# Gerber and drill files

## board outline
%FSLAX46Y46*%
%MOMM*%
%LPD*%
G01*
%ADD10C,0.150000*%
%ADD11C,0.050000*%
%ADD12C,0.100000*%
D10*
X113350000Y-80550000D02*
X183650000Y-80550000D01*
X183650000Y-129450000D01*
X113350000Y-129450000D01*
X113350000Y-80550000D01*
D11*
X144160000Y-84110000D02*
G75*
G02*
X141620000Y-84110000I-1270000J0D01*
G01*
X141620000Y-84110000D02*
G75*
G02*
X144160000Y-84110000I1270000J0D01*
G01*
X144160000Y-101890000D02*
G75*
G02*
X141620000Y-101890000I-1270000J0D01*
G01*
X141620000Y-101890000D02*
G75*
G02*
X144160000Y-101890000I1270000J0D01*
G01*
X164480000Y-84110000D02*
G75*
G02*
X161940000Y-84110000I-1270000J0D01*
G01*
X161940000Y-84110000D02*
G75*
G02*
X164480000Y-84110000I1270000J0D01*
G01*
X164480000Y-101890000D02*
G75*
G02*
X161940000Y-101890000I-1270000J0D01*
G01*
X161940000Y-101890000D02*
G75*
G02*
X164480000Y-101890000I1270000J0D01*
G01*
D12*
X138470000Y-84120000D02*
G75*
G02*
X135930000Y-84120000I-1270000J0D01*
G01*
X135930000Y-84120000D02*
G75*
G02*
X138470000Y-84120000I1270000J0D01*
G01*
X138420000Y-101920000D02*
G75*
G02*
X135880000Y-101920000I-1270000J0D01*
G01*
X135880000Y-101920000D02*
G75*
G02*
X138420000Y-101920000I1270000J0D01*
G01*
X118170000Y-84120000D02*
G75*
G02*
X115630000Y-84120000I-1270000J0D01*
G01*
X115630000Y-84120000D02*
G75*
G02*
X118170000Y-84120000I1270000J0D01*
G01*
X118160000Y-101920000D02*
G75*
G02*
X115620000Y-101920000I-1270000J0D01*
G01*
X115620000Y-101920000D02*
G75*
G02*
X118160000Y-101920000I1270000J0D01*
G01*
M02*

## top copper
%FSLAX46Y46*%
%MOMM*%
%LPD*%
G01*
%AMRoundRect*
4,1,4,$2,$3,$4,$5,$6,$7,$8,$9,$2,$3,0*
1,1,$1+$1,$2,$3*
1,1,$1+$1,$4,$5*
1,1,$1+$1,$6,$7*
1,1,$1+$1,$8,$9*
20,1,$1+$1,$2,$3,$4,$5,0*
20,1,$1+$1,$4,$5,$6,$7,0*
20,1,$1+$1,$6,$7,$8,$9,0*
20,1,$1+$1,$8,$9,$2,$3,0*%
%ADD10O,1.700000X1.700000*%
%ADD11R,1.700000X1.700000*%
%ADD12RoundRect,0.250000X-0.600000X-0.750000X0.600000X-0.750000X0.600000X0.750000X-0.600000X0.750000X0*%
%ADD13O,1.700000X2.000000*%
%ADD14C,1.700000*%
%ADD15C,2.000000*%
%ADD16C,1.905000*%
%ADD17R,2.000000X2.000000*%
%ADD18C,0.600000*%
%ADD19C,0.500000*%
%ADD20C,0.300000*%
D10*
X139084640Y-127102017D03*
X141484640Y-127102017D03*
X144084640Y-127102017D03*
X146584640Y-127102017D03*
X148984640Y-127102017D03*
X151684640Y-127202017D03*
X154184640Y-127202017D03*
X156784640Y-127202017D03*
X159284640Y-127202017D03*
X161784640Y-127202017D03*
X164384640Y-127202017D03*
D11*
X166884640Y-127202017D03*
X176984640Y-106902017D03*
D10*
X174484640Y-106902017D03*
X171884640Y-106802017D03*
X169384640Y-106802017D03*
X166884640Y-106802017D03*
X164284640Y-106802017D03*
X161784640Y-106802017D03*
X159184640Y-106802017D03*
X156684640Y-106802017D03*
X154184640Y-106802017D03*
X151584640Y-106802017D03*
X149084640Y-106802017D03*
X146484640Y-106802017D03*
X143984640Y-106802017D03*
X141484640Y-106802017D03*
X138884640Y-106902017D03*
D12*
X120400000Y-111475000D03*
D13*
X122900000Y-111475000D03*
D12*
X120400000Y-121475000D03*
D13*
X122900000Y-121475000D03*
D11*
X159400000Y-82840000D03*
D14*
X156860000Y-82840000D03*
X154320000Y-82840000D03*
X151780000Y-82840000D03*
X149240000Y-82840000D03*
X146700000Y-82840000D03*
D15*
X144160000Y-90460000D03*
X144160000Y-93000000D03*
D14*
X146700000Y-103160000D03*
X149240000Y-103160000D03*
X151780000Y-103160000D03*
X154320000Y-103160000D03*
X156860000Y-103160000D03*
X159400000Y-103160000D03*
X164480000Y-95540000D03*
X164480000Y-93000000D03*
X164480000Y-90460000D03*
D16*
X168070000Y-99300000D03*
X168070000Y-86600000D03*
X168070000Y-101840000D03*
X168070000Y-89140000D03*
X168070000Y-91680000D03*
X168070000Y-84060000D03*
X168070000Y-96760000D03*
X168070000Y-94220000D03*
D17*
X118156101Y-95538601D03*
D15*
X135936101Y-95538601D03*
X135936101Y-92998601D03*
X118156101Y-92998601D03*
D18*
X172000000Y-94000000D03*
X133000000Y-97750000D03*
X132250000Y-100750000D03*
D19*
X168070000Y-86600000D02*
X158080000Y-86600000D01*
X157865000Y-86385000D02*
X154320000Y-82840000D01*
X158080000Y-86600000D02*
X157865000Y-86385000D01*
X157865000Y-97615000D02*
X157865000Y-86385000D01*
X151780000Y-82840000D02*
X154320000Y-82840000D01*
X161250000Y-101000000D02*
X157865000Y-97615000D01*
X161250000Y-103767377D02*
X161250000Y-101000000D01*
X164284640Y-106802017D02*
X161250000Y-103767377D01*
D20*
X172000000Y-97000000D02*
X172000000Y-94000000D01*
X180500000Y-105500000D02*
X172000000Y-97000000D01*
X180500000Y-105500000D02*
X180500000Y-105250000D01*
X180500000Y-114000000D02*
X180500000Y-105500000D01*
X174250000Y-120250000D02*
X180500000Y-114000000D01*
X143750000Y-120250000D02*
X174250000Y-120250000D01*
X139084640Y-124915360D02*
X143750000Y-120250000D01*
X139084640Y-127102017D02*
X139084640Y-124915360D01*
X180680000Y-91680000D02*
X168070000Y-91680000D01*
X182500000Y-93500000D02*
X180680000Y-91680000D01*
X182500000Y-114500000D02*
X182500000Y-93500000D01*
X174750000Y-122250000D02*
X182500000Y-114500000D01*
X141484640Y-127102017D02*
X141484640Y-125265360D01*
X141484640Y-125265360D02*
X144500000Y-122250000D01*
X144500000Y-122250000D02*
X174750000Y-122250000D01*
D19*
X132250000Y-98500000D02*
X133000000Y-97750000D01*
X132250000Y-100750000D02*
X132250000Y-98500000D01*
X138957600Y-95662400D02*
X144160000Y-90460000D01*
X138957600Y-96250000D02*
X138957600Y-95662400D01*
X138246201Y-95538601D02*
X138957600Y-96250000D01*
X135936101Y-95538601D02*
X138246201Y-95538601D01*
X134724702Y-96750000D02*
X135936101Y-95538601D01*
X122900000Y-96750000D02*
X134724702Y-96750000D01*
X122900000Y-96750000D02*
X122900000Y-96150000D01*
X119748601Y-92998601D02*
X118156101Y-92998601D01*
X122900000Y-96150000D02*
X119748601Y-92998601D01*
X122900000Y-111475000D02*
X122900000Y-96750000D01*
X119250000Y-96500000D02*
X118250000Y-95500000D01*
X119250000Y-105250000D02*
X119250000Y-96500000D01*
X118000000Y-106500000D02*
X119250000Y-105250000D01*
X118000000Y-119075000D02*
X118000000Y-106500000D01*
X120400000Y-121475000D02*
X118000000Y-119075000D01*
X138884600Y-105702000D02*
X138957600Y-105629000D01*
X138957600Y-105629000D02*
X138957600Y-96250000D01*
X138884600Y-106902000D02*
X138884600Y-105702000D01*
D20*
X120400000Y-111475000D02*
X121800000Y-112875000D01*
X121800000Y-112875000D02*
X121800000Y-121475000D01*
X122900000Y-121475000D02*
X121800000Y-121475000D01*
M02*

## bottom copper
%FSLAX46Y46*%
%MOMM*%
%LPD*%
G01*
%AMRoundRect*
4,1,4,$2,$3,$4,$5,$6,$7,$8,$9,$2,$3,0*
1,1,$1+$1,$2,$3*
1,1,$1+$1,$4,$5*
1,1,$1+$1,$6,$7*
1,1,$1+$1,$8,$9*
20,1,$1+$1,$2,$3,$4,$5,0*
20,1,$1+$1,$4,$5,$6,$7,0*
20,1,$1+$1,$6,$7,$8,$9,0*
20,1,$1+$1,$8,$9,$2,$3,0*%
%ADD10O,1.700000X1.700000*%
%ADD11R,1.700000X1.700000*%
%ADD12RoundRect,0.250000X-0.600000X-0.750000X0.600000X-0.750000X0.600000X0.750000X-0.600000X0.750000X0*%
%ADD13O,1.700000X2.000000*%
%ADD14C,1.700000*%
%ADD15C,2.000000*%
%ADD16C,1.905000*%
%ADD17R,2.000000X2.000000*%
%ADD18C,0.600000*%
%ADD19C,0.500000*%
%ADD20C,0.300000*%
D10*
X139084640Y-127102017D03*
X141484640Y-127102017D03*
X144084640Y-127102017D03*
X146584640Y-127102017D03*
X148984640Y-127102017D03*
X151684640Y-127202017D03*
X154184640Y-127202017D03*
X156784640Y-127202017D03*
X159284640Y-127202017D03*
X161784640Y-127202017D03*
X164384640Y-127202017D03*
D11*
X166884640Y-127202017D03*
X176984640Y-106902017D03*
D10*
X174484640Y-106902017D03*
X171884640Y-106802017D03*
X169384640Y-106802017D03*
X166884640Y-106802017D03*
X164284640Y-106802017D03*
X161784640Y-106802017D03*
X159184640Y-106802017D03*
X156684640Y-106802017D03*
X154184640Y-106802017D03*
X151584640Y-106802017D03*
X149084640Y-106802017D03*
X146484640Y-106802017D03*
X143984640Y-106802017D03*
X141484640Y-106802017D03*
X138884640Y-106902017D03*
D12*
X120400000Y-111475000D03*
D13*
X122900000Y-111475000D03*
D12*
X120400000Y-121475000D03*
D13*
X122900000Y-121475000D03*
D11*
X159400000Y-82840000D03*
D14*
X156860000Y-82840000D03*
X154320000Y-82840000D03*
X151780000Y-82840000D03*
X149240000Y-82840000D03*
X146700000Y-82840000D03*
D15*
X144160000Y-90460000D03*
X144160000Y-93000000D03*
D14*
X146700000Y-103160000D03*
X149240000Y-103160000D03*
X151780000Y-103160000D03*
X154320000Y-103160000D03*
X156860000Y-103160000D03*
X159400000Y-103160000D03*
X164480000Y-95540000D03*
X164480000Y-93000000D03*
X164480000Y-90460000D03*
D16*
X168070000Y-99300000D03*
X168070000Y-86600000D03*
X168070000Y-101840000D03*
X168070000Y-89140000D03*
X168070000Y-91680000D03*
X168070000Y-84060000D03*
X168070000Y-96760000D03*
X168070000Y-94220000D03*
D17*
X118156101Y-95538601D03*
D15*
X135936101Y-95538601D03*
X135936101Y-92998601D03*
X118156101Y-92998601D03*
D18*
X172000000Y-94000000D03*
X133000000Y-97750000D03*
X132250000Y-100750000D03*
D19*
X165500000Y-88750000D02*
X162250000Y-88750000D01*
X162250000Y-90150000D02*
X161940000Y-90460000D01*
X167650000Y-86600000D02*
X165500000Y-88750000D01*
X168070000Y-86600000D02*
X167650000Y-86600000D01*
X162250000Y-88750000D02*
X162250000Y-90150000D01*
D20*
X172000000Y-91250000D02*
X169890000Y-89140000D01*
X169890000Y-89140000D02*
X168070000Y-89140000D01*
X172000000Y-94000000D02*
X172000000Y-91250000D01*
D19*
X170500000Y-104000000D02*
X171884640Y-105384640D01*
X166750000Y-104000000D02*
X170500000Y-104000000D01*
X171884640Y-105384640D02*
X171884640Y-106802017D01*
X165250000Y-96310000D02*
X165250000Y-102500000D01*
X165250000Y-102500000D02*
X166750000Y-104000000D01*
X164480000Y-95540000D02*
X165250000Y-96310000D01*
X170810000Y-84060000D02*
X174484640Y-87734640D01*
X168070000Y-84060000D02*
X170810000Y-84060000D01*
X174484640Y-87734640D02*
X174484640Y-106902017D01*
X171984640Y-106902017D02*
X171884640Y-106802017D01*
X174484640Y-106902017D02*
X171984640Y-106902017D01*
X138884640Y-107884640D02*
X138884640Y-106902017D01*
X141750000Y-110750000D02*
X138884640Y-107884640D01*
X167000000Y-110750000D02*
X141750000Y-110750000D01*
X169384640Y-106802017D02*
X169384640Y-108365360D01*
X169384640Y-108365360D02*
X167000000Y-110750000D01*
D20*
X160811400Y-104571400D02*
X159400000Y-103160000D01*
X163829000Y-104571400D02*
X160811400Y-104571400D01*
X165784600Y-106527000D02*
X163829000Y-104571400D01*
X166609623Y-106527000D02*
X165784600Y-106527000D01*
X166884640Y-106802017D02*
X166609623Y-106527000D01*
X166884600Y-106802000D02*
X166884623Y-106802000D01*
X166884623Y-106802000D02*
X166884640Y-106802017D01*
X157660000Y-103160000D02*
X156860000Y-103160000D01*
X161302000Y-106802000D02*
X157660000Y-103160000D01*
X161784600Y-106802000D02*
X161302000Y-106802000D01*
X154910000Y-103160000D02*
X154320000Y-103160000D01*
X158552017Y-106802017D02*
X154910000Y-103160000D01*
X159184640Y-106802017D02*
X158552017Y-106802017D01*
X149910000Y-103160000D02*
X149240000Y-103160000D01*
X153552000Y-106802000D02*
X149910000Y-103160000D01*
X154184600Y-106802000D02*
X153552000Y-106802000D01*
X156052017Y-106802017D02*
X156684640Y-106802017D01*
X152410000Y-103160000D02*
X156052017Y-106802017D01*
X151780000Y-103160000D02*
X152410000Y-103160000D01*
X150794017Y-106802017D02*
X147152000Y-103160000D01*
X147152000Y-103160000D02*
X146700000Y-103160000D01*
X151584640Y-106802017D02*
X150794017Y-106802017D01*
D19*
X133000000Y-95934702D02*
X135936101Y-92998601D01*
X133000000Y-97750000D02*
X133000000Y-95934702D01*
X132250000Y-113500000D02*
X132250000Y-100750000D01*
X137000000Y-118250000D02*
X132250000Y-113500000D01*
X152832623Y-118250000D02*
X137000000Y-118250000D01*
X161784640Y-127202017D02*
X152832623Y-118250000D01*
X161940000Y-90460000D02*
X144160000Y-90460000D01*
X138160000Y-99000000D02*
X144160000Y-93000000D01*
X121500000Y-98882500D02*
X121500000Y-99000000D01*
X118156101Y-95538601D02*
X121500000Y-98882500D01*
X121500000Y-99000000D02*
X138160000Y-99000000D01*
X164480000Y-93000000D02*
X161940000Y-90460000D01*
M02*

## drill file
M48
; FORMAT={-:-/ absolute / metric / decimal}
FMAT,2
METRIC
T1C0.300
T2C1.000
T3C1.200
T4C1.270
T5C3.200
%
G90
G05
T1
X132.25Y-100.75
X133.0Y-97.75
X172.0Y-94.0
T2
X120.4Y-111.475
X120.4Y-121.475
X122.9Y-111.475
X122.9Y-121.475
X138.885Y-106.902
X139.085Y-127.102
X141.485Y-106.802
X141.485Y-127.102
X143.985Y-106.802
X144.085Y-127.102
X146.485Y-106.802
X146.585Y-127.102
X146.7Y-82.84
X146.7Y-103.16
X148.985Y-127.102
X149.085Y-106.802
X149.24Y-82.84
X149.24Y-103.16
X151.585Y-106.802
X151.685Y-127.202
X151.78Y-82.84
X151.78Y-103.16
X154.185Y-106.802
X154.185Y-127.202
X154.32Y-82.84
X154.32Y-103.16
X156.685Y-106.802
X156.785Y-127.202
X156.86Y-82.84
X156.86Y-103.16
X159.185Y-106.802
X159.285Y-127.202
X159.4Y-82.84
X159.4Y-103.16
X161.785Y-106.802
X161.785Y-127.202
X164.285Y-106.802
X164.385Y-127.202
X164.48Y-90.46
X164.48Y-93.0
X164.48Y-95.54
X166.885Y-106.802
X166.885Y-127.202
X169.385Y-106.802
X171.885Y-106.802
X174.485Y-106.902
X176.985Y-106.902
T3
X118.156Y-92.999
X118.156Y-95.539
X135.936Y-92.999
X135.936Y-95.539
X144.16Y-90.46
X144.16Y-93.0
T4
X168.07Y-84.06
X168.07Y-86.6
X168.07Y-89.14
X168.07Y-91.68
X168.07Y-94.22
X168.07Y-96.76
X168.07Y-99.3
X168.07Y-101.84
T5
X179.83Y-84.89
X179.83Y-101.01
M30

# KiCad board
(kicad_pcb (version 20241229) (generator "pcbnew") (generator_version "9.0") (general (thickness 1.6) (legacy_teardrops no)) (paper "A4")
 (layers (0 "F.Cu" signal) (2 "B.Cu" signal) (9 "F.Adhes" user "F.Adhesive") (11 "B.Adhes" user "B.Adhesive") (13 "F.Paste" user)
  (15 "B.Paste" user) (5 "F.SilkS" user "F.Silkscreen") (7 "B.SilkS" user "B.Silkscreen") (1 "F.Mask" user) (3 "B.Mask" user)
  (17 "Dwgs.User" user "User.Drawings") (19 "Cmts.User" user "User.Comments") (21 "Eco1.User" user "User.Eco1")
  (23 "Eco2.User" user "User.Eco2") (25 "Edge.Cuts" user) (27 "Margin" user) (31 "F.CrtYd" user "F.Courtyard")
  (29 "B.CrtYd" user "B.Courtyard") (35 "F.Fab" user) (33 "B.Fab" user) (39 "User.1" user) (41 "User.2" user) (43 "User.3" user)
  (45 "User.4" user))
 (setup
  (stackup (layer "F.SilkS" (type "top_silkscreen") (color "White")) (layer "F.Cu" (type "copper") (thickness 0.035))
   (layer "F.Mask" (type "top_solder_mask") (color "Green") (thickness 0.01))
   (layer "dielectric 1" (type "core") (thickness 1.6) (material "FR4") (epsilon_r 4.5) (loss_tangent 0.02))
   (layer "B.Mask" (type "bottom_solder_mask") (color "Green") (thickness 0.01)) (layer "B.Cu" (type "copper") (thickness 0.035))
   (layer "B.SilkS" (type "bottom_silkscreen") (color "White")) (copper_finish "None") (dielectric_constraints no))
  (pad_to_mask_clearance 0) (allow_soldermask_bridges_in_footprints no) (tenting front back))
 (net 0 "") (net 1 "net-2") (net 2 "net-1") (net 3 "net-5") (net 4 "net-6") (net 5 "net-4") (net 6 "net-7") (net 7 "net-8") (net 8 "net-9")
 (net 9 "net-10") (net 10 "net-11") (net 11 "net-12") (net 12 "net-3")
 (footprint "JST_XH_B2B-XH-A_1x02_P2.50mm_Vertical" (layer "F.Cu") (at 121.65 112)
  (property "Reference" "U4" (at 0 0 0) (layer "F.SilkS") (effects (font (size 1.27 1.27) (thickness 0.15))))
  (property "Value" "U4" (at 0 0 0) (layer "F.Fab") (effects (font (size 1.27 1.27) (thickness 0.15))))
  (pad "1" thru_hole roundrect (at -1.25 -0.525) (size 1.7 2) (drill 1) (layers "*.Cu" "*.Mask") (remove_unused_layers no)
   (roundrect_rratio 0.147059) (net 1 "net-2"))
  (pad "2" thru_hole oval (at 1.25 -0.525) (size 1.7 2) (drill 1) (layers "*.Cu" "*.Mask") (remove_unused_layers no) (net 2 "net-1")))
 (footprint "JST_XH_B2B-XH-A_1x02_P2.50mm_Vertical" (layer "F.Cu") (at 121.65 122)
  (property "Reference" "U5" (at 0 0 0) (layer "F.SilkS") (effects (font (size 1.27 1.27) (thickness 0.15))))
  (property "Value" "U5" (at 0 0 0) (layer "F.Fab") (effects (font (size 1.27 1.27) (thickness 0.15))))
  (pad "1" thru_hole roundrect (at -1.25 -0.525) (size 1.7 2) (drill 1) (layers "*.Cu" "*.Mask") (remove_unused_layers no)
   (roundrect_rratio 0.147059) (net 2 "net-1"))
  (pad "2" thru_hole oval (at 1.25 -0.525) (size 1.7 2) (drill 1) (layers "*.Cu" "*.Mask") (remove_unused_layers no) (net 1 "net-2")))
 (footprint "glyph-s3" (layer "F.Cu") (at 157.978 117.1 180)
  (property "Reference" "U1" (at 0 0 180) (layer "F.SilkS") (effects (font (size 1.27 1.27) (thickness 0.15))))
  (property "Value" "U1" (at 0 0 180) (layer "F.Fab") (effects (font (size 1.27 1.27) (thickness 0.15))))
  (pad "1" thru_hole oval (at 18.89336 -10.002017 270) (size 1.7 1.7) (drill 1) (layers "*.Cu" "*.Mask") (remove_unused_layers no))
  (pad "2" thru_hole oval (at 16.49336 -10.002017 270) (size 1.7 1.7) (drill 1) (layers "*.Cu" "*.Mask") (remove_unused_layers no))
  (pad "3" thru_hole oval (at 13.89336 -10.002017 270) (size 1.7 1.7) (drill 1) (layers "*.Cu" "*.Mask") (remove_unused_layers no)
   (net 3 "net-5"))
  (pad "4" thru_hole oval (at 11.39336 -10.002017 270) (size 1.7 1.7) (drill 1) (layers "*.Cu" "*.Mask") (remove_unused_layers no)
   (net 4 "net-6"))
  (pad "5" thru_hole oval (at 8.99336 -10.002017 270) (size 1.7 1.7) (drill 1) (layers "*.Cu" "*.Mask") (remove_unused_layers no))
  (pad "6" thru_hole oval (at 6.29336 -10.102017 270) (size 1.7 1.7) (drill 1) (layers "*.Cu" "*.Mask") (remove_unused_layers no))
  (pad "7" thru_hole oval (at 3.79336 -10.102017 270) (size 1.7 1.7) (drill 1) (layers "*.Cu" "*.Mask") (remove_unused_layers no))
  (pad "8" thru_hole oval (at 1.19336 -10.102017 270) (size 1.7 1.7) (drill 1) (layers "*.Cu" "*.Mask") (remove_unused_layers no))
  (pad "9" thru_hole oval (at -1.30664 -10.102017 270) (size 1.7 1.7) (drill 1) (layers "*.Cu" "*.Mask") (remove_unused_layers no))
  (pad "10" thru_hole oval (at -3.80664 -10.102017 270) (size 1.7 1.7) (drill 1) (layers "*.Cu" "*.Mask") (remove_unused_layers no)
   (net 2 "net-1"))
  (pad "11" thru_hole oval (at -6.40664 -10.102017 270) (size 1.7 1.7) (drill 1) (layers "*.Cu" "*.Mask") (remove_unused_layers no))
  (pad "12" thru_hole rect (at -8.90664 -10.102017 270) (size 1.7 1.7) (drill 1) (layers "*.Cu" "*.Mask") (remove_unused_layers no))
  (pad "13" thru_hole rect (at -19.00664 10.197983 270) (size 1.7 1.7) (drill 1) (layers "*.Cu" "*.Mask") (remove_unused_layers no))
  (pad "14" thru_hole oval (at -16.50664 10.197983 270) (size 1.7 1.7) (drill 1) (layers "*.Cu" "*.Mask") (remove_unused_layers no)
   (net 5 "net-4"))
  (pad "15" thru_hole oval (at -13.90664 10.297983 270) (size 1.7 1.7) (drill 1) (layers "*.Cu" "*.Mask") (remove_unused_layers no)
   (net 5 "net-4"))
  (pad "16" thru_hole oval (at -11.40664 10.297983 270) (size 1.7 1.7) (drill 1) (layers "*.Cu" "*.Mask") (remove_unused_layers no)
   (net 2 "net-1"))
  (pad "17" thru_hole oval (at -8.90664 10.297983 270) (size 1.7 1.7) (drill 1) (layers "*.Cu" "*.Mask") (remove_unused_layers no)
   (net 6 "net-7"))
  (pad "18" thru_hole oval (at -6.30664 10.297983 270) (size 1.7 1.7) (drill 1) (layers "*.Cu" "*.Mask") (remove_unused_layers no))
  (pad "19" thru_hole oval (at -3.80664 10.297983 270) (size 1.7 1.7) (drill 1) (layers "*.Cu" "*.Mask") (remove_unused_layers no)
   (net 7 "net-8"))
  (pad "20" thru_hole oval (at -1.20664 10.297983 270) (size 1.7 1.7) (drill 1) (layers "*.Cu" "*.Mask") (remove_unused_layers no)
   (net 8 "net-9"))
  (pad "21" thru_hole oval (at 1.29336 10.297983 270) (size 1.7 1.7) (drill 1) (layers "*.Cu" "*.Mask") (remove_unused_layers no)
   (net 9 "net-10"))
  (pad "22" thru_hole oval (at 3.79336 10.297983 270) (size 1.7 1.7) (drill 1) (layers "*.Cu" "*.Mask") (remove_unused_layers no)
   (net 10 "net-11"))
  (pad "23" thru_hole oval (at 6.39336 10.297983 270) (size 1.7 1.7) (drill 1) (layers "*.Cu" "*.Mask") (remove_unused_layers no)
   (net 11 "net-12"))
  (pad "24" thru_hole oval (at 8.89336 10.297983 270) (size 1.7 1.7) (drill 1) (layers "*.Cu" "*.Mask") (remove_unused_layers no))
  (pad "25" thru_hole oval (at 11.49336 10.297983 270) (size 1.7 1.7) (drill 1) (layers "*.Cu" "*.Mask") (remove_unused_layers no))
  (pad "26" thru_hole oval (at 13.99336 10.297983 270) (size 1.7 1.7) (drill 1) (layers "*.Cu" "*.Mask") (remove_unused_layers no))
  (pad "27" thru_hole oval (at 16.49336 10.297983 270) (size 1.7 1.7) (drill 1) (layers "*.Cu" "*.Mask") (remove_unused_layers no))
  (pad "28" thru_hole oval (at 19.09336 10.197983 270) (size 1.7 1.7) (drill 1) (layers "*.Cu" "*.Mask") (remove_unused_layers no)
   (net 2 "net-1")))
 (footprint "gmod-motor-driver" (layer "F.Cu") (at 153.05 93)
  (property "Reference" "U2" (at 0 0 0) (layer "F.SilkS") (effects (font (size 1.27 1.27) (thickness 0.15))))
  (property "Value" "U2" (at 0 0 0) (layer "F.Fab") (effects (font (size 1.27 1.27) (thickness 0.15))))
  (fp_circle (center -10.16 -8.89) (end -10.16 -10.16) (stroke (width 0.05) (type default)) (fill no) (layer "Edge.Cuts"))
  (fp_circle (center -10.16 8.89) (end -10.16 7.62) (stroke (width 0.05) (type default)) (fill no) (layer "Edge.Cuts"))
  (fp_circle (center 10.16 -8.89) (end 10.16 -10.16) (stroke (width 0.05) (type default)) (fill no) (layer "Edge.Cuts"))
  (fp_circle (center 10.16 8.89) (end 10.16 7.62) (stroke (width 0.05) (type default)) (fill no) (layer "Edge.Cuts"))
  (pad "1" thru_hole rect (at 6.35 -10.16 270) (size 1.7 1.7) (drill 1) (layers "*.Cu" "*.Mask") (remove_unused_layers no))
  (pad "2" thru_hole circle (at 3.81 -10.16 270) (size 1.7 1.7) (drill 1) (layers "*.Cu" "*.Mask") (remove_unused_layers no))
  (pad "3" thru_hole circle (at 1.27 -10.16 270) (size 1.7 1.7) (drill 1) (layers "*.Cu" "*.Mask") (remove_unused_layers no))
  (pad "4" thru_hole circle (at -1.27 -10.16 270) (size 1.7 1.7) (drill 1) (layers "*.Cu" "*.Mask") (remove_unused_layers no))
  (pad "5" thru_hole circle (at -3.81 -10.16 270) (size 1.7 1.7) (drill 1) (layers "*.Cu" "*.Mask") (remove_unused_layers no))
  (pad "6" thru_hole circle (at -6.35 -10.16 270) (size 1.7 1.7) (drill 1) (layers "*.Cu" "*.Mask") (remove_unused_layers no))
  (pad "7" thru_hole circle (at -8.89 -2.54 270) (size 2 2) (drill 1.2) (layers "*.Cu" "*.Mask") (remove_unused_layers no) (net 2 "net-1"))
  (pad "8" thru_hole circle (at -8.89 0 270) (size 2 2) (drill 1.2) (layers "*.Cu" "*.Mask") (remove_unused_layers no) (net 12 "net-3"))
  (pad "9" thru_hole circle (at -6.35 10.16 270) (size 1.7 1.7) (drill 1) (layers "*.Cu" "*.Mask") (remove_unused_layers no)
   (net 11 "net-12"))
  (pad "10" thru_hole circle (at -3.81 10.16 270) (size 1.7 1.7) (drill 1) (layers "*.Cu" "*.Mask") (remove_unused_layers no)
   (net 10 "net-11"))
  (pad "11" thru_hole circle (at -1.27 10.16 270) (size 1.7 1.7) (drill 1) (layers "*.Cu" "*.Mask") (remove_unused_layers no)
   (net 9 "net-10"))
  (pad "12" thru_hole circle (at 1.27 10.16 270) (size 1.7 1.7) (drill 1) (layers "*.Cu" "*.Mask") (remove_unused_layers no) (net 8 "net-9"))
  (pad "13" thru_hole circle (at 3.81 10.16 270) (size 1.7 1.7) (drill 1) (layers "*.Cu" "*.Mask") (remove_unused_layers no) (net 7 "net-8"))
  (pad "14" thru_hole circle (at 6.35 10.16 270) (size 1.7 1.7) (drill 1) (layers "*.Cu" "*.Mask") (remove_unused_layers no) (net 6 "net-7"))
  (pad "15" thru_hole circle (at 11.43 2.54 180) (size 1.7 1.7) (drill 1) (layers "*.Cu" "*.Mask") (remove_unused_layers no) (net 5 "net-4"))
  (pad "16" thru_hole circle (at 11.43 0 180) (size 1.7 1.7) (drill 1) (layers "*.Cu" "*.Mask") (remove_unused_layers no) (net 2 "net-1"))
  (pad "17" thru_hole circle (at 11.43 -2.54 180) (size 1.7 1.7) (drill 1) (layers "*.Cu" "*.Mask") (remove_unused_layers no)))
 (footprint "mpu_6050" (layer "F.Cu") (at 174.4 92.95)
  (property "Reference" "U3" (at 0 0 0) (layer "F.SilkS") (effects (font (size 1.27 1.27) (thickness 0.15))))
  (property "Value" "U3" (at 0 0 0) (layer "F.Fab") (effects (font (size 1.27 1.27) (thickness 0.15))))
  (pad "" np_thru_hole circle (at 5.43 -8.06) (size 3.2 3.2) (drill 3.2) (layers "*.Cu" "*.Mask"))
  (pad "" np_thru_hole circle (at 5.43 8.06) (size 3.2 3.2) (drill 3.2) (layers "*.Cu" "*.Mask"))
  (pad "AD0" thru_hole circle (at -6.33 6.35) (size 1.905 1.905) (drill 1.27) (layers "*.Cu" "*.Mask") (remove_unused_layers no)
   (solder_mask_margin 0.102))
  (pad "GND" thru_hole circle (at -6.33 -6.35) (size 1.905 1.905) (drill 1.27) (layers "*.Cu" "*.Mask") (remove_unused_layers no)
   (solder_mask_margin 0.102))
  (pad "INT" thru_hole circle (at -6.33 8.89) (size 1.905 1.905) (drill 1.27) (layers "*.Cu" "*.Mask") (remove_unused_layers no)
   (solder_mask_margin 0.102))
  (pad "SCL" thru_hole circle (at -6.33 -3.81) (size 1.905 1.905) (drill 1.27) (layers "*.Cu" "*.Mask") (remove_unused_layers no)
   (solder_mask_margin 0.102))
  (pad "SDA" thru_hole circle (at -6.33 -1.27) (size 1.905 1.905) (drill 1.27) (layers "*.Cu" "*.Mask") (remove_unused_layers no)
   (solder_mask_margin 0.102))
  (pad "VCC" thru_hole circle (at -6.33 -8.89) (size 1.905 1.905) (drill 1.27) (layers "*.Cu" "*.Mask") (remove_unused_layers no)
   (solder_mask_margin 0.102))
  (pad "XCL" thru_hole circle (at -6.33 3.81) (size 1.905 1.905) (drill 1.27) (layers "*.Cu" "*.Mask") (remove_unused_layers no)
   (solder_mask_margin 0.102))
  (pad "XDA" thru_hole circle (at -6.33 1.27) (size 1.905 1.905) (drill 1.27) (layers "*.Cu" "*.Mask") (remove_unused_layers no)
   (solder_mask_margin 0.102)))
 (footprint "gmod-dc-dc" (layer "F.Cu") (at 127.05 93 180)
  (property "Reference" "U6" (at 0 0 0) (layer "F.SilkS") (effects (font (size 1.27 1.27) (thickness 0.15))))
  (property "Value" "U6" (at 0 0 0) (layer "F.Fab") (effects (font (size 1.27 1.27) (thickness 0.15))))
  (fp_circle (center 10.16 -8.92) (end 11.43 -8.92) (stroke (width 0.1) (type solid)) (fill no) (layer "Edge.Cuts"))
  (fp_circle (center 10.15 8.88) (end 11.42 8.88) (stroke (width 0.1) (type solid)) (fill no) (layer "Edge.Cuts"))
  (fp_circle (center -10.1 -8.92) (end -8.83 -8.92) (stroke (width 0.1) (type solid)) (fill no) (layer "Edge.Cuts"))
  (fp_circle (center -10.15 8.88) (end -8.88 8.88) (stroke (width 0.1) (type solid)) (fill no) (layer "Edge.Cuts"))
  (pad "1" thru_hole rect (at 8.893899 -2.538601 270) (size 2 2) (drill 1.2) (layers "*.Cu" "*.Mask") (remove_unused_layers no))
  (pad "2" thru_hole circle (at -8.886101 -2.538601 90) (size 2 2) (drill 1.2) (layers "*.Cu" "*.Mask") (remove_unused_layers no)
   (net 2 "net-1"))
  (pad "3" thru_hole circle (at -8.886101 0.001399 90) (size 2 2) (drill 1.2) (layers "*.Cu" "*.Mask") (remove_unused_layers no)
   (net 2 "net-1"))
  (pad "4" thru_hole circle (at 8.893899 0.001399 270) (size 2 2) (drill 1.2) (layers "*.Cu" "*.Mask") (remove_unused_layers no)
   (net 2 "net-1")))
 (gr_rect (start 113.35 80.55) (end 183.65 129.45) (stroke (width 0.15) (type solid)) (fill no) (layer "Edge.Cuts"))
 (segment (start 139.08464 127.102017) (end 139.08464 124.91536) (width 0.3) (layer "F.Cu") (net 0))
 (segment (start 144.5 122.25) (end 174.75 122.25) (width 0.3) (layer "F.Cu") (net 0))
 (segment (start 180.5 105.5) (end 172 97) (width 0.3) (layer "F.Cu") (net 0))
 (segment (start 174.75 122.25) (end 182.5 114.5) (width 0.3) (layer "F.Cu") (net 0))
 (segment (start 180.5 114) (end 180.5 105.5) (width 0.3) (layer "F.Cu") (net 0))
 (segment (start 182.5 93.5) (end 180.68 91.68) (width 0.3) (layer "F.Cu") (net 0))
 (segment (start 139.08464 124.91536) (end 143.75 120.25) (width 0.3) (layer "F.Cu") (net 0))
 (segment (start 141.48464 127.102017) (end 141.48464 125.26536) (width 0.3) (layer "F.Cu") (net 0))
 (segment (start 141.48464 125.26536) (end 144.5 122.25) (width 0.3) (layer "F.Cu") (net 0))
 (segment (start 143.75 120.25) (end 174.25 120.25) (width 0.3) (layer "F.Cu") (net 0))
 (segment (start 180.68 91.68) (end 168.07 91.68) (width 0.3) (layer "F.Cu") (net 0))
 (segment (start 180.5 105.5) (end 180.5 105.25) (width 0.3) (layer "F.Cu") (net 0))
 (segment (start 174.25 120.25) (end 180.5 114) (width 0.3) (layer "F.Cu") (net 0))
 (segment (start 172 97) (end 172 94) (width 0.3) (layer "F.Cu") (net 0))
 (segment (start 182.5 114.5) (end 182.5 93.5) (width 0.3) (layer "F.Cu") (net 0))
 (via (at 172 94) (size 0.6) (drill 0.3) (layers "F.Cu" "B.Cu") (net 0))
 (segment (start 121.5 98.8825) (end 121.5 99) (width 0.5) (layer "B.Cu") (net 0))
 (segment (start 169.89 89.14) (end 168.07 89.14) (width 0.3) (layer "B.Cu") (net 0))
 (segment (start 118.156101 95.538601) (end 121.5 98.8825) (width 0.5) (layer "B.Cu") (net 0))
 (segment (start 172 94) (end 172 91.25) (width 0.3) (layer "B.Cu") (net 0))
 (segment (start 172 91.25) (end 169.89 89.14) (width 0.3) (layer "B.Cu") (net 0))
 (segment (start 161.25 101) (end 157.865 97.615) (width 0.5) (layer "F.Cu") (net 2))
 (segment (start 157.865 86.385) (end 154.32 82.84) (width 0.5) (layer "F.Cu") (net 2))
 (segment (start 157.865 97.615) (end 157.865 86.385) (width 0.5) (layer "F.Cu") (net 2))
 (segment (start 135.936101 95.538601) (end 138.246201 95.538601) (width 0.5) (layer "F.Cu") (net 2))
 (segment (start 134.724702 96.75) (end 135.936101 95.538601) (width 0.5) (layer "F.Cu") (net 2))
 (segment (start 122.9 96.15) (end 119.748601 92.998601) (width 0.5) (layer "F.Cu") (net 2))
 (segment (start 119.748601 92.998601) (end 118.156101 92.998601) (width 0.5) (layer "F.Cu") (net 2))
 (segment (start 119.25 105.25) (end 119.25 96.5) (width 0.5) (layer "F.Cu") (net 2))
 (segment (start 120.4 121.475) (end 118 119.075) (width 0.5) (layer "F.Cu") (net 2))
 (segment (start 122.9 96.75) (end 134.724702 96.75) (width 0.5) (layer "F.Cu") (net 2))
 (segment (start 158.08 86.6) (end 157.865 86.385) (width 0.5) (layer "F.Cu") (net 2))
 (segment (start 132.25 98.5) (end 133 97.75) (width 0.5) (layer "F.Cu") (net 2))
 (segment (start 164.28464 106.802017) (end 161.25 103.767377) (width 0.5) (layer "F.Cu") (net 2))
 (segment (start 122.9 96.75) (end 122.9 96.15) (width 0.5) (layer "F.Cu") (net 2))
 (segment (start 138.9576 95.6624) (end 144.16 90.46) (width 0.5) (layer "F.Cu") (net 2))
 (segment (start 168.07 86.6) (end 158.08 86.6) (width 0.5) (layer "F.Cu") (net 2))
 (segment (start 138.246201 95.538601) (end 138.9576 96.25) (width 0.5) (layer "F.Cu") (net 2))
 (segment (start 161.25 103.767377) (end 161.25 101) (width 0.5) (layer "F.Cu") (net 2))
 (segment (start 138.8846 105.702) (end 138.9576 105.629) (width 0.5) (layer "F.Cu") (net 2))
 (segment (start 118 119.075) (end 118 106.5) (width 0.5) (layer "F.Cu") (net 2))
 (segment (start 132.25 100.75) (end 132.25 98.5) (width 0.5) (layer "F.Cu") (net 2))
 (segment (start 119.25 96.5) (end 118.25 95.5) (width 0.5) (layer "F.Cu") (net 2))
 (segment (start 118 106.5) (end 119.25 105.25) (width 0.5) (layer "F.Cu") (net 2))
 (segment (start 122.9 111.475) (end 122.9 96.75) (width 0.5) (layer "F.Cu") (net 2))
 (segment (start 138.9576 96.25) (end 138.9576 95.6624) (width 0.5) (layer "F.Cu") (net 2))
 (segment (start 151.78 82.84) (end 154.32 82.84) (width 0.5) (layer "F.Cu") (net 2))
 (segment (start 138.9576 105.629) (end 138.9576 96.25) (width 0.5) (layer "F.Cu") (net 2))
 (segment (start 138.8846 106.902) (end 138.8846 105.702) (width 0.5) (layer "F.Cu") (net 2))
 (via (at 133 97.75) (size 0.6) (drill 0.3) (layers "F.Cu" "B.Cu") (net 2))
 (via (at 132.25 100.75) (size 0.6) (drill 0.3) (layers "F.Cu" "B.Cu") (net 2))
 (segment (start 165.5 88.75) (end 162.25 88.75) (width 0.5) (layer "B.Cu") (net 2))
 (segment (start 161.94 90.46) (end 144.16 90.46) (width 0.5) (layer "B.Cu") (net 2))
 (segment (start 137 118.25) (end 132.25 113.5) (width 0.5) (layer "B.Cu") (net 2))
 (segment (start 133 97.75) (end 133 95.934702) (width 0.5) (layer "B.Cu") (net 2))
 (segment (start 162.25 90.15) (end 161.94 90.46) (width 0.5) (layer "B.Cu") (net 2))
 (segment (start 164.48 93) (end 161.94 90.46) (width 0.5) (layer "B.Cu") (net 2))
 (segment (start 138.88464 107.88464) (end 138.88464 106.902017) (width 0.5) (layer "B.Cu") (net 2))
 (segment (start 169.38464 106.802017) (end 169.38464 108.36536) (width 0.5) (layer "B.Cu") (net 2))
 (segment (start 141.75 110.75) (end 138.88464 107.88464) (width 0.5) (layer "B.Cu") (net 2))
 (segment (start 168.07 86.6) (end 167.65 86.6) (width 0.5) (layer "B.Cu") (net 2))
 (segment (start 133 95.934702) (end 135.936101 92.998601) (width 0.5) (layer "B.Cu") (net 2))
 (segment (start 169.38464 108.36536) (end 167 110.75) (width 0.5) (layer "B.Cu") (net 2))
 (segment (start 167.65 86.6) (end 165.5 88.75) (width 0.5) (layer "B.Cu") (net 2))
 (segment (start 152.832623 118.25) (end 137 118.25) (width 0.5) (layer "B.Cu") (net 2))
 (segment (start 162.25 88.75) (end 162.25 90.15) (width 0.5) (layer "B.Cu") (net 2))
 (segment (start 132.25 113.5) (end 132.25 100.75) (width 0.5) (layer "B.Cu") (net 2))
 (segment (start 161.78464 127.202017) (end 152.832623 118.25) (width 0.5) (layer "B.Cu") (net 2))
 (segment (start 167 110.75) (end 141.75 110.75) (width 0.5) (layer "B.Cu") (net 2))
 (segment (start 120.4 111.475) (end 121.8 112.875) (width 0.3) (layer "F.Cu") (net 1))
 (segment (start 121.8 112.875) (end 121.8 121.475) (width 0.3) (layer "F.Cu") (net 1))
 (segment (start 122.9 121.475) (end 121.8 121.475) (width 0.3) (layer "F.Cu") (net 1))
 (segment (start 138.16 99) (end 144.16 93) (width 0.5) (layer "B.Cu") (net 12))
 (segment (start 121.5 99) (end 138.16 99) (width 0.5) (layer "B.Cu") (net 12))
 (segment (start 170.81 84.06) (end 174.48464 87.73464) (width 0.5) (layer "B.Cu") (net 5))
 (segment (start 164.48 95.54) (end 165.25 96.31) (width 0.5) (layer "B.Cu") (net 5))
 (segment (start 166.75 104) (end 170.5 104) (width 0.5) (layer "B.Cu") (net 5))
 (segment (start 170.5 104) (end 171.88464 105.38464) (width 0.5) (layer "B.Cu") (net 5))
 (segment (start 174.48464 87.73464) (end 174.48464 106.902017) (width 0.5) (layer "B.Cu") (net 5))
 (segment (start 168.07 84.06) (end 170.81 84.06) (width 0.5) (layer "B.Cu") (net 5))
 (segment (start 165.25 102.5) (end 166.75 104) (width 0.5) (layer "B.Cu") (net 5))
 (segment (start 165.25 96.31) (end 165.25 102.5) (width 0.5) (layer "B.Cu") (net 5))
 (segment (start 171.88464 105.38464) (end 171.88464 106.802017) (width 0.5) (layer "B.Cu") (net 5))
 (segment (start 171.98464 106.902017) (end 171.88464 106.802017) (width 0.5) (layer "B.Cu") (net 5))
 (segment (start 174.48464 106.902017) (end 171.98464 106.902017) (width 0.5) (layer "B.Cu") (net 5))
 (segment (start 166.609623 106.527) (end 165.7846 106.527) (width 0.3) (layer "B.Cu") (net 6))
 (segment (start 160.8114 104.5714) (end 159.4 103.16) (width 0.3) (layer "B.Cu") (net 6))
 (segment (start 166.884623 106.802) (end 166.88464 106.802017) (width 0.3) (layer "B.Cu") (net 6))
 (segment (start 165.7846 106.527) (end 163.829 104.5714) (width 0.3) (layer "B.Cu") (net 6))
 (segment (start 166.8846 106.802) (end 166.884623 106.802) (width 0.3) (layer "B.Cu") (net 6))
 (segment (start 166.88464 106.802017) (end 166.609623 106.527) (width 0.3) (layer "B.Cu") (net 6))
 (segment (start 163.829 104.5714) (end 160.8114 104.5714) (width 0.3) (layer "B.Cu") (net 6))
 (segment (start 161.7846 106.802) (end 161.302 106.802) (width 0.3) (layer "B.Cu") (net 7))
 (segment (start 161.302 106.802) (end 157.66 103.16) (width 0.3) (layer "B.Cu") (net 7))
 (segment (start 157.66 103.16) (end 156.86 103.16) (width 0.3) (layer "B.Cu") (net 7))
 (segment (start 154.91 103.16) (end 154.32 103.16) (width 0.3) (layer "B.Cu") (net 8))
 (segment (start 159.18464 106.802017) (end 158.552017 106.802017) (width 0.3) (layer "B.Cu") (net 8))
 (segment (start 158.552017 106.802017) (end 154.91 103.16) (width 0.3) (layer "B.Cu") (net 8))
 (segment (start 151.78 103.16) (end 152.41 103.16) (width 0.3) (layer "B.Cu") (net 9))
 (segment (start 152.41 103.16) (end 156.052017 106.802017) (width 0.3) (layer "B.Cu") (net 9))
 (segment (start 156.052017 106.802017) (end 156.68464 106.802017) (width 0.3) (layer "B.Cu") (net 9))
 (segment (start 154.1846 106.802) (end 153.552 106.802) (width 0.3) (layer "B.Cu") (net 10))
 (segment (start 153.552 106.802) (end 149.91 103.16) (width 0.3) (layer "B.Cu") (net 10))
 (segment (start 149.91 103.16) (end 149.24 103.16) (width 0.3) (layer "B.Cu") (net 10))
 (segment (start 151.58464 106.802017) (end 150.794017 106.802017) (width 0.3) (layer "B.Cu") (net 11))
 (segment (start 147.152 103.16) (end 146.7 103.16) (width 0.3) (layer "B.Cu") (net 11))
 (segment (start 150.794017 106.802017) (end 147.152 103.16) (width 0.3) (layer "B.Cu") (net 11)))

